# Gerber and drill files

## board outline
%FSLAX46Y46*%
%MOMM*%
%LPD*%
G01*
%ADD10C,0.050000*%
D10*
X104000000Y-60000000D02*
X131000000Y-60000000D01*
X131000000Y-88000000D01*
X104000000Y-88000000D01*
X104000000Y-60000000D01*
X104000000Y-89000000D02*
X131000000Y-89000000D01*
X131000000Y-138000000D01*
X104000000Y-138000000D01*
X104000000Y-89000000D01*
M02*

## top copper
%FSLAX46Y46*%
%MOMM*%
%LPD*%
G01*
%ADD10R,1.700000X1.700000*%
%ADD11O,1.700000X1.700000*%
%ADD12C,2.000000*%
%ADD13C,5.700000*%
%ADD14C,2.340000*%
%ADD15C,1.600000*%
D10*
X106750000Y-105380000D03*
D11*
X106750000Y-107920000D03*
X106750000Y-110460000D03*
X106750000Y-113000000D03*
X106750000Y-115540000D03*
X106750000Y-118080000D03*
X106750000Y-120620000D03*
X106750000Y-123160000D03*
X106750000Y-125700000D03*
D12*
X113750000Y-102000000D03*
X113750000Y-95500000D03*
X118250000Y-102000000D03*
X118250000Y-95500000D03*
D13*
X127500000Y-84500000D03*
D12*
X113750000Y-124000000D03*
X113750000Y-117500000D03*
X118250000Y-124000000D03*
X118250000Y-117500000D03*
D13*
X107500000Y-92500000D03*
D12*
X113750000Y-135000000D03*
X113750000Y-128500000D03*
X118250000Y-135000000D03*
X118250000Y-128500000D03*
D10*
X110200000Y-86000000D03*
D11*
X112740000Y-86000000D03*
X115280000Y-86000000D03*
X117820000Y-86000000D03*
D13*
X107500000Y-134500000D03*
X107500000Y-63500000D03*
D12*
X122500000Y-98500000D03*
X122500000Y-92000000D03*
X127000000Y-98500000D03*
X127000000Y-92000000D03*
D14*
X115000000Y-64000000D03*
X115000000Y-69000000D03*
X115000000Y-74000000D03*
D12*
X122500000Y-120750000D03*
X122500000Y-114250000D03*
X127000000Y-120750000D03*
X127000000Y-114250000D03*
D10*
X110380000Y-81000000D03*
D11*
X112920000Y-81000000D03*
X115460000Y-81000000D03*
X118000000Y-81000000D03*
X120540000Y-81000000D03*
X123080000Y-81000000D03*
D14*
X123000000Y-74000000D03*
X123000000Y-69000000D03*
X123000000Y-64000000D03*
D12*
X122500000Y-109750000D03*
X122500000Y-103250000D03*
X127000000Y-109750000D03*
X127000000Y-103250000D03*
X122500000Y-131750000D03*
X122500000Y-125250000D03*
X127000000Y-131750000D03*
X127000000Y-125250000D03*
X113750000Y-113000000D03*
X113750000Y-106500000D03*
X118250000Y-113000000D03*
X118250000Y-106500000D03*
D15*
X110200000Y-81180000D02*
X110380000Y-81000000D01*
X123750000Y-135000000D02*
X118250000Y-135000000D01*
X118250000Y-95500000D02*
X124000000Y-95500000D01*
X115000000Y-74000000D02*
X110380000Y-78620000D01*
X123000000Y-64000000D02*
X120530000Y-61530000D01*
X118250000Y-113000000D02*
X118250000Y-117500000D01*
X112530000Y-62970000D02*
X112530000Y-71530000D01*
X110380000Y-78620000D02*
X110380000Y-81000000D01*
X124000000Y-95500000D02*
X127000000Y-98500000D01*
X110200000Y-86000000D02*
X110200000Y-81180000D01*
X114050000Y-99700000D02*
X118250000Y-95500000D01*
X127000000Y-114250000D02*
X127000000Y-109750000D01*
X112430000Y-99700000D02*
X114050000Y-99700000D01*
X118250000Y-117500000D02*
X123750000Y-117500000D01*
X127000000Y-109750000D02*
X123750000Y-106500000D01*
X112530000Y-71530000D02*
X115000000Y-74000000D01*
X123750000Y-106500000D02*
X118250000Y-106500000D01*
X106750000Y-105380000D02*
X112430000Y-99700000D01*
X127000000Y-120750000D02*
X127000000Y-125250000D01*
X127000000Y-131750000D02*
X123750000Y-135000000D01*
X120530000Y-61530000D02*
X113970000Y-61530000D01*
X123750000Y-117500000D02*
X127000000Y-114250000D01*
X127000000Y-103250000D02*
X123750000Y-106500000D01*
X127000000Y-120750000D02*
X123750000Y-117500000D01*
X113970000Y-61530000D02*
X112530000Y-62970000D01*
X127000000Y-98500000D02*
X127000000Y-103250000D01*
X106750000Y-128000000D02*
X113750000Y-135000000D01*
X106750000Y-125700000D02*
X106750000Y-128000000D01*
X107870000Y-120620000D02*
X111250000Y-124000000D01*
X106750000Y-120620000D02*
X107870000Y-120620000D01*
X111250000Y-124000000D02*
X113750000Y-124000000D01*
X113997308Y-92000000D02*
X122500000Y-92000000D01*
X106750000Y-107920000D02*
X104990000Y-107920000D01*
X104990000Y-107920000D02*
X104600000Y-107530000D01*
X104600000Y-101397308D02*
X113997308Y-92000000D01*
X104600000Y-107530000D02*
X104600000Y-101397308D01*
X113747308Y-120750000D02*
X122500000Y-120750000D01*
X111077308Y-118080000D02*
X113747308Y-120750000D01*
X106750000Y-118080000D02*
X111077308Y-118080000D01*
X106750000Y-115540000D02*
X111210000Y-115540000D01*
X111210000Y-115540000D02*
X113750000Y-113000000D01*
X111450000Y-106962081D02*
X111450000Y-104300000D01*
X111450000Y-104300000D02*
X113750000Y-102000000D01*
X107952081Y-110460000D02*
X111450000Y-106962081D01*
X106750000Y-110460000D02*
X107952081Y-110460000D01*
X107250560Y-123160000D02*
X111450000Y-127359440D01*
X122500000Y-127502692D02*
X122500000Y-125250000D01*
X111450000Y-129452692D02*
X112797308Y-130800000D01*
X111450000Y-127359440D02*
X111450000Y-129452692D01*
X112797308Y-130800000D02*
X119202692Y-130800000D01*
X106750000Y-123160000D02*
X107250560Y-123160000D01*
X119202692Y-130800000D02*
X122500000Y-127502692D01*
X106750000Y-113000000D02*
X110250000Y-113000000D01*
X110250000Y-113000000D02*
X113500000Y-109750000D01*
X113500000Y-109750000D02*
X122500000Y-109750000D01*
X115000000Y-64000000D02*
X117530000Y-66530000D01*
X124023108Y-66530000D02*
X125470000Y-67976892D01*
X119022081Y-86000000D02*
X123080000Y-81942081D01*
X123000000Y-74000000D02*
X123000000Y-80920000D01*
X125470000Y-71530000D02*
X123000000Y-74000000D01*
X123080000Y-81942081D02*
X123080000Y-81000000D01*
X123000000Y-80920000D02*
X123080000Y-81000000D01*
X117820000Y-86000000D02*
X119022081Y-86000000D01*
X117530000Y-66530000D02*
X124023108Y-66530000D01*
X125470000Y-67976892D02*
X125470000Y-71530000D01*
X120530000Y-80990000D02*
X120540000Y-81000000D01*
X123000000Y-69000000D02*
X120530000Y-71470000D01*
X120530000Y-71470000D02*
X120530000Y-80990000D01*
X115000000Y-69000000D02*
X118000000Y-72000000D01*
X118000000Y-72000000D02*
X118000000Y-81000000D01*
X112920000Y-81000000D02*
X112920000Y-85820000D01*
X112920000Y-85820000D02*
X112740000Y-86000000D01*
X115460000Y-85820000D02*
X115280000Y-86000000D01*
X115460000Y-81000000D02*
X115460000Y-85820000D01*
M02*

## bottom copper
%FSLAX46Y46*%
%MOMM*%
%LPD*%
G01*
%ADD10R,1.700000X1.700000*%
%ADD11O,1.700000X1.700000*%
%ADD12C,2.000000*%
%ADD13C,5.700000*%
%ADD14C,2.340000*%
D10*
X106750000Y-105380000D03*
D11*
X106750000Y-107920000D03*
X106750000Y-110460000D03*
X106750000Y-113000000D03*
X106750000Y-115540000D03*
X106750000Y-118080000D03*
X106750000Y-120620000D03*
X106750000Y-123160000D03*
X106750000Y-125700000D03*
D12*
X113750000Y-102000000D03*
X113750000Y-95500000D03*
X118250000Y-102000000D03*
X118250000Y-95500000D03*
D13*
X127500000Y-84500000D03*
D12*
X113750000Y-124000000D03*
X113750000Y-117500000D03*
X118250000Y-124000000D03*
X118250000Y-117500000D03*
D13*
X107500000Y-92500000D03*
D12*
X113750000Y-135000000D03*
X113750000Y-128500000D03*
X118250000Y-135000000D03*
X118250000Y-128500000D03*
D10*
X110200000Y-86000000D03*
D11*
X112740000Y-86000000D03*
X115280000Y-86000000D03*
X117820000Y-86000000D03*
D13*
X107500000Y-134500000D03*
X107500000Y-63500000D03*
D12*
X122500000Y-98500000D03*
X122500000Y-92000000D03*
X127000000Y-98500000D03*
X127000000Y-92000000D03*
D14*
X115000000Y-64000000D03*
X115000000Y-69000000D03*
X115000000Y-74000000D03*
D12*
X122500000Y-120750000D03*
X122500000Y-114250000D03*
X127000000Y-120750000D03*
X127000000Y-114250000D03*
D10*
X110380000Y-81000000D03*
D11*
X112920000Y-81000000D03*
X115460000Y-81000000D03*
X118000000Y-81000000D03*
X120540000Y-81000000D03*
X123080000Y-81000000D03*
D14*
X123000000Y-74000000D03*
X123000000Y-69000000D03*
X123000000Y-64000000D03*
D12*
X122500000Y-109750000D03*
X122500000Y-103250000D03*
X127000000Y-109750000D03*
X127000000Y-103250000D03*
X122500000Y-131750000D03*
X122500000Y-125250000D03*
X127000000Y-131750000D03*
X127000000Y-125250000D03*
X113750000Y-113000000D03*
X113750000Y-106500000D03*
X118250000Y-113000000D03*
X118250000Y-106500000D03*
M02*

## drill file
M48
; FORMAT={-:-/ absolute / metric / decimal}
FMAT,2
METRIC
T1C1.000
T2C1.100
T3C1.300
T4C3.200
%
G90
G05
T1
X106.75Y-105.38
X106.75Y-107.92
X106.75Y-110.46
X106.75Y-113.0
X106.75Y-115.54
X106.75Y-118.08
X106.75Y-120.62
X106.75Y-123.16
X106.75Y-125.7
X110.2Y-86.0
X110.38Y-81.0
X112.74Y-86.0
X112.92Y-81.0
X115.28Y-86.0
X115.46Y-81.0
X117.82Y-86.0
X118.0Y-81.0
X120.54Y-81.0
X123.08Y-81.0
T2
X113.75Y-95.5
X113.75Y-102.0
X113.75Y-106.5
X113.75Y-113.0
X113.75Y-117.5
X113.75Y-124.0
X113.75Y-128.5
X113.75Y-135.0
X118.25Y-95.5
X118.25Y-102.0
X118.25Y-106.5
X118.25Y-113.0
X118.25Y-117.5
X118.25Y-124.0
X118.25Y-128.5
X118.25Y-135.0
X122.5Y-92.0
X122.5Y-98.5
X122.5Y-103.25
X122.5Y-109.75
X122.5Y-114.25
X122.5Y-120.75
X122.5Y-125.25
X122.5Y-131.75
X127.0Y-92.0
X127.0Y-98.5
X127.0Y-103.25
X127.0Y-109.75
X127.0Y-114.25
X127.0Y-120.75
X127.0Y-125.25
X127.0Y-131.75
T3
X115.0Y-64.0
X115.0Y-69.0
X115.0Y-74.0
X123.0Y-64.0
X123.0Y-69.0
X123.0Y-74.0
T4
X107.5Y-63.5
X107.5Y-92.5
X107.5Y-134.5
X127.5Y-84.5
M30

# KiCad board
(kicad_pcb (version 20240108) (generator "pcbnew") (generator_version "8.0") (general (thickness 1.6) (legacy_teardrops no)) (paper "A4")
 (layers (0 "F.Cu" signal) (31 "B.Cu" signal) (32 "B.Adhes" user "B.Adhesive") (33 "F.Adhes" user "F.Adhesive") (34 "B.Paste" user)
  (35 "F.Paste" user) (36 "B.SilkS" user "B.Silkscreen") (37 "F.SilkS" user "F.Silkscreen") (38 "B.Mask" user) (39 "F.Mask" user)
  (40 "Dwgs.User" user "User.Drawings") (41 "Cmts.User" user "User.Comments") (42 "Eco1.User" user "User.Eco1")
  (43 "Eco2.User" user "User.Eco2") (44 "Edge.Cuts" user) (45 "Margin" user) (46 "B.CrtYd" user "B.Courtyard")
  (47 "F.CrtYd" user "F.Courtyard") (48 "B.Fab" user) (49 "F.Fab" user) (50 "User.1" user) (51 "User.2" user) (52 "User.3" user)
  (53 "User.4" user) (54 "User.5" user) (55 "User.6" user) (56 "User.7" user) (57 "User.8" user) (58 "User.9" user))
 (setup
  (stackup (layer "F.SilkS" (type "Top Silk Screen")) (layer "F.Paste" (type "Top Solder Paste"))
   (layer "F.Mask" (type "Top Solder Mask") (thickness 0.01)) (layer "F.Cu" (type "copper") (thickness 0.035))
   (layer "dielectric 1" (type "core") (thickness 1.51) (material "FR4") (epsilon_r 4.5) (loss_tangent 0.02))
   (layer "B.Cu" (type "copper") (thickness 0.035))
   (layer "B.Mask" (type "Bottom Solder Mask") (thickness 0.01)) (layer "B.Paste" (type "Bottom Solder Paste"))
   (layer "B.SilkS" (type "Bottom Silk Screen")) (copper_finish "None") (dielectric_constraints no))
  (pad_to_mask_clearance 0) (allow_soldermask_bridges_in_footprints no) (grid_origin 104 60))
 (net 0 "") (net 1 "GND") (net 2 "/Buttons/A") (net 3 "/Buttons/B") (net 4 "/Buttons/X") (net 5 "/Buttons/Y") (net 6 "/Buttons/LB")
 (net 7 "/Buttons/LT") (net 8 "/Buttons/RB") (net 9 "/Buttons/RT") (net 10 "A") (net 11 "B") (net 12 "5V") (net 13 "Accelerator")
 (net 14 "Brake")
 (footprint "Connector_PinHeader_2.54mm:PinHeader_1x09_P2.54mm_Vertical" (layer "F.Cu") (at 106.75 105.38)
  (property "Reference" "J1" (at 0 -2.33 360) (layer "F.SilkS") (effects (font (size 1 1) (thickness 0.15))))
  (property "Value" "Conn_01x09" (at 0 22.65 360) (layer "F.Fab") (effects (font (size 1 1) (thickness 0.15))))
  (pad "1" thru_hole rect (at 0 0) (size 1.7 1.7) (drill 1) (layers "*.Cu" "*.Mask") (remove_unused_layers no) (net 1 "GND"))
  (pad "2" thru_hole oval (at 0 2.54) (size 1.7 1.7) (drill 1) (layers "*.Cu" "*.Mask") (remove_unused_layers no) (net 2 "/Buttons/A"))
  (pad "3" thru_hole oval (at 0 5.08) (size 1.7 1.7) (drill 1) (layers "*.Cu" "*.Mask") (remove_unused_layers no) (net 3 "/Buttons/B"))
  (pad "4" thru_hole oval (at 0 7.62) (size 1.7 1.7) (drill 1) (layers "*.Cu" "*.Mask") (remove_unused_layers no) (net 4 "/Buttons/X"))
  (pad "5" thru_hole oval (at 0 10.16) (size 1.7 1.7) (drill 1) (layers "*.Cu" "*.Mask") (remove_unused_layers no) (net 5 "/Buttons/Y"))
  (pad "6" thru_hole oval (at 0 12.7) (size 1.7 1.7) (drill 1) (layers "*.Cu" "*.Mask") (remove_unused_layers no) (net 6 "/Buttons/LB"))
  (pad "7" thru_hole oval (at 0 15.24) (size 1.7 1.7) (drill 1) (layers "*.Cu" "*.Mask") (remove_unused_layers no) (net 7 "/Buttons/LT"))
  (pad "8" thru_hole oval (at 0 17.78) (size 1.7 1.7) (drill 1) (layers "*.Cu" "*.Mask") (remove_unused_layers no) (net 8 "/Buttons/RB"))
  (pad "9" thru_hole oval (at 0 20.32) (size 1.7 1.7) (drill 1) (layers "*.Cu" "*.Mask") (remove_unused_layers no) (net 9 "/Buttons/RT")))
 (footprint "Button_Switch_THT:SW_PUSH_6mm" (layer "F.Cu") (at 113.75 102 90)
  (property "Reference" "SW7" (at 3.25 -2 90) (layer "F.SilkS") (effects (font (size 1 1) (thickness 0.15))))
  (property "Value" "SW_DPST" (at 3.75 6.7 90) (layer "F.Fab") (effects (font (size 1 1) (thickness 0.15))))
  (pad "1" thru_hole circle (at 0 0 180) (size 2 2) (drill 1.1) (layers "*.Cu" "*.Mask") (remove_unused_layers no) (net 3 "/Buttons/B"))
  (pad "1" thru_hole circle (at 6.5 0 180) (size 2 2) (drill 1.1) (layers "*.Cu" "*.Mask") (remove_unused_layers no) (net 3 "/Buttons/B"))
  (pad "2" thru_hole circle (at 0 4.5 180) (size 2 2) (drill 1.1) (layers "*.Cu" "*.Mask") (remove_unused_layers no) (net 1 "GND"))
  (pad "2" thru_hole circle (at 6.5 4.5 180) (size 2 2) (drill 1.1) (layers "*.Cu" "*.Mask") (remove_unused_layers no) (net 1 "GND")))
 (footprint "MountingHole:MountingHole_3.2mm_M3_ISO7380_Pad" (layer "F.Cu") (at 127.5 84.5)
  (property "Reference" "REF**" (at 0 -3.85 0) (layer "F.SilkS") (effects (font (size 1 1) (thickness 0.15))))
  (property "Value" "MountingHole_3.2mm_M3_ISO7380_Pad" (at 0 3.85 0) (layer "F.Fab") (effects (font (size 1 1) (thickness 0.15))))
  (pad "1" thru_hole circle (at 0 0) (size 5.7 5.7) (drill 3.2) (layers "*.Cu" "*.Mask") (remove_unused_layers no)))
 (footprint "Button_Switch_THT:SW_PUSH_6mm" (layer "F.Cu") (at 113.75 124 90)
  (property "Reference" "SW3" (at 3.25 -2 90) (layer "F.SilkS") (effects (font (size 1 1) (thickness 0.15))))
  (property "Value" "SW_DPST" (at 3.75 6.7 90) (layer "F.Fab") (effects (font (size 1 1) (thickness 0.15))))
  (pad "1" thru_hole circle (at 0 0 180) (size 2 2) (drill 1.1) (layers "*.Cu" "*.Mask") (remove_unused_layers no) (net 7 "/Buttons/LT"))
  (pad "1" thru_hole circle (at 6.5 0 180) (size 2 2) (drill 1.1) (layers "*.Cu" "*.Mask") (remove_unused_layers no) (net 7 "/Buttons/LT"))
  (pad "2" thru_hole circle (at 0 4.5 180) (size 2 2) (drill 1.1) (layers "*.Cu" "*.Mask") (remove_unused_layers no) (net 1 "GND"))
  (pad "2" thru_hole circle (at 6.5 4.5 180) (size 2 2) (drill 1.1) (layers "*.Cu" "*.Mask") (remove_unused_layers no) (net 1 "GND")))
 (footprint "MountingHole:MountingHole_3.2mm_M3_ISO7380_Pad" (layer "F.Cu") (at 107.5 92.5)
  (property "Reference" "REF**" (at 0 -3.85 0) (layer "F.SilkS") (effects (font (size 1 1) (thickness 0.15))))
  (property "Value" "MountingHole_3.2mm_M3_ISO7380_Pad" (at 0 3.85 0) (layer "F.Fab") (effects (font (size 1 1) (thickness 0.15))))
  (pad "1" thru_hole circle (at 0 0) (size 5.7 5.7) (drill 3.2) (layers "*.Cu" "*.Mask") (remove_unused_layers no)))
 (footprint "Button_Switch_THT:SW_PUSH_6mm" (layer "F.Cu") (at 113.75 135 90)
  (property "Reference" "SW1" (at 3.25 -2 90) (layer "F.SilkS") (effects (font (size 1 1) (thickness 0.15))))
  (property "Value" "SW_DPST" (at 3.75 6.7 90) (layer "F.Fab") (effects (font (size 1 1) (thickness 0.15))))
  (pad "1" thru_hole circle (at 0 0 180) (size 2 2) (drill 1.1) (layers "*.Cu" "*.Mask") (remove_unused_layers no) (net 9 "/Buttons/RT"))
  (pad "1" thru_hole circle (at 6.5 0 180) (size 2 2) (drill 1.1) (layers "*.Cu" "*.Mask") (remove_unused_layers no) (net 9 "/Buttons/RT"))
  (pad "2" thru_hole circle (at 0 4.5 180) (size 2 2) (drill 1.1) (layers "*.Cu" "*.Mask") (remove_unused_layers no) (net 1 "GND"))
  (pad "2" thru_hole circle (at 6.5 4.5 180) (size 2 2) (drill 1.1) (layers "*.Cu" "*.Mask") (remove_unused_layers no) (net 1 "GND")))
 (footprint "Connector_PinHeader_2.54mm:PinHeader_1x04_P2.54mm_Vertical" (layer "F.Cu") (at 110.2 86 90)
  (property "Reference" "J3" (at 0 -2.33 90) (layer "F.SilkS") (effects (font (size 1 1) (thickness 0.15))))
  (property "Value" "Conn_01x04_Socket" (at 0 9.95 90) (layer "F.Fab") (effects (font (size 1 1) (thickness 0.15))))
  (pad "1" thru_hole rect (at 0 0 90) (size 1.7 1.7) (drill 1) (layers "*.Cu" "*.Mask") (remove_unused_layers no) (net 1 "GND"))
  (pad "2" thru_hole oval (at 0 2.54 90) (size 1.7 1.7) (drill 1) (layers "*.Cu" "*.Mask") (remove_unused_layers no) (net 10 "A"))
  (pad "3" thru_hole oval (at 0 5.08 90) (size 1.7 1.7) (drill 1) (layers "*.Cu" "*.Mask") (remove_unused_layers no) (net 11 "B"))
  (pad "4" thru_hole oval (at 0 7.62 90) (size 1.7 1.7) (drill 1) (layers "*.Cu" "*.Mask") (remove_unused_layers no) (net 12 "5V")))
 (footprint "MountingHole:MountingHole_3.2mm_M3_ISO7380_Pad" (layer "F.Cu") (at 107.5 134.5)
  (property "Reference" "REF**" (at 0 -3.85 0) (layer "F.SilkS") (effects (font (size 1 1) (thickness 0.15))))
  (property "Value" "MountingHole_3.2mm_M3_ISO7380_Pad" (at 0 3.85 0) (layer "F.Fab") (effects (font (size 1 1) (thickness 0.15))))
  (pad "1" thru_hole circle (at 0 0) (size 5.7 5.7) (drill 3.2) (layers "*.Cu" "*.Mask") (remove_unused_layers no)))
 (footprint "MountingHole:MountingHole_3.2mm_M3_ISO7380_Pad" (layer "F.Cu") (at 107.5 63.5)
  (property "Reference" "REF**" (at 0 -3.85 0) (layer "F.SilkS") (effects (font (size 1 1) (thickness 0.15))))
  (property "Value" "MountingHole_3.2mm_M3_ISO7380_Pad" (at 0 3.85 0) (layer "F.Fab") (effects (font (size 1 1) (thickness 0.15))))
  (pad "1" thru_hole circle (at 0 0) (size 5.7 5.7) (drill 3.2) (layers "*.Cu" "*.Mask") (remove_unused_layers no)))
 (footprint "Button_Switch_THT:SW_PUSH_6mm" (layer "F.Cu") (at 122.5 98.5 90)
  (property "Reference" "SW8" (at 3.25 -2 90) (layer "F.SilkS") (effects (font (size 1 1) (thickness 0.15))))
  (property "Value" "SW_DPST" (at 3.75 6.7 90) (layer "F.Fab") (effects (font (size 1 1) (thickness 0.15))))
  (pad "1" thru_hole circle (at 0 0 180) (size 2 2) (drill 1.1) (layers "*.Cu" "*.Mask") (remove_unused_layers no) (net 2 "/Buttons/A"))
  (pad "1" thru_hole circle (at 6.5 0 180) (size 2 2) (drill 1.1) (layers "*.Cu" "*.Mask") (remove_unused_layers no) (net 2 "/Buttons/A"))
  (pad "2" thru_hole circle (at 0 4.5 180) (size 2 2) (drill 1.1) (layers "*.Cu" "*.Mask") (remove_unused_layers no) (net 1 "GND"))
  (pad "2" thru_hole circle (at 6.5 4.5 180) (size 2 2) (drill 1.1) (layers "*.Cu" "*.Mask") (remove_unused_layers no) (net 1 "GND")))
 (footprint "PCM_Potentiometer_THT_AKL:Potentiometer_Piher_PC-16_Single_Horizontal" (layer "F.Cu") (at 115 64 180)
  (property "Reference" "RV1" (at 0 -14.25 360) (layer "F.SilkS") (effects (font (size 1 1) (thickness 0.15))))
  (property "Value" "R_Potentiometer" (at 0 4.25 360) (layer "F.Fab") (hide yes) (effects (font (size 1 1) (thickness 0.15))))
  (pad "1" thru_hole circle (at 0 0 180) (size 2.34 2.34) (drill 1.3) (layers "*.Cu" "*.Mask") (remove_unused_layers no) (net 12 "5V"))
  (pad "2" thru_hole circle (at 0 -5 180) (size 2.34 2.34) (drill 1.3) (layers "*.Cu" "*.Mask") (remove_unused_layers no)
   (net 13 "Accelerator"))
  (pad "3" thru_hole circle (at 0 -10 180) (size 2.34 2.34) (drill 1.3) (layers "*.Cu" "*.Mask") (remove_unused_layers no) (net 1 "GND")))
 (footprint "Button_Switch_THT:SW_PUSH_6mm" (layer "F.Cu") (at 122.5 120.75 90)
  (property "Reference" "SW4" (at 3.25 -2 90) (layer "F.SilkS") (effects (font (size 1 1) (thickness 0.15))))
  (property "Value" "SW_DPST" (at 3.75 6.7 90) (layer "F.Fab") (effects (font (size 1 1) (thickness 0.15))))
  (pad "1" thru_hole circle (at 0 0 180) (size 2 2) (drill 1.1) (layers "*.Cu" "*.Mask") (remove_unused_layers no) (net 6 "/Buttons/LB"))
  (pad "1" thru_hole circle (at 6.5 0 180) (size 2 2) (drill 1.1) (layers "*.Cu" "*.Mask") (remove_unused_layers no) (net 6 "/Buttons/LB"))
  (pad "2" thru_hole circle (at 0 4.5 180) (size 2 2) (drill 1.1) (layers "*.Cu" "*.Mask") (remove_unused_layers no) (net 1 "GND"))
  (pad "2" thru_hole circle (at 6.5 4.5 180) (size 2 2) (drill 1.1) (layers "*.Cu" "*.Mask") (remove_unused_layers no) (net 1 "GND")))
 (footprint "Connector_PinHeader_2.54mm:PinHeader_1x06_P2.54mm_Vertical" (layer "F.Cu") (at 110.38 81 90)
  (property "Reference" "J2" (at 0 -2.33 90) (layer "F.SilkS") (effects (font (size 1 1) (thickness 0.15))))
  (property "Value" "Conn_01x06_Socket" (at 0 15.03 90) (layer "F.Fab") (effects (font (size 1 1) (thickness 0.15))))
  (pad "1" thru_hole rect (at 0 0 90) (size 1.7 1.7) (drill 1) (layers "*.Cu" "*.Mask") (remove_unused_layers no) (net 1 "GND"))
  (pad "2" thru_hole oval (at 0 2.54 90) (size 1.7 1.7) (drill 1) (layers "*.Cu" "*.Mask") (remove_unused_layers no) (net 10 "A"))
  (pad "3" thru_hole oval (at 0 5.08 90) (size 1.7 1.7) (drill 1) (layers "*.Cu" "*.Mask") (remove_unused_layers no) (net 11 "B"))
  (pad "4" thru_hole oval (at 0 7.62 90) (size 1.7 1.7) (drill 1) (layers "*.Cu" "*.Mask") (remove_unused_layers no) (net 13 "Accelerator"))
  (pad "5" thru_hole oval (at 0 10.16 90) (size 1.7 1.7) (drill 1) (layers "*.Cu" "*.Mask") (remove_unused_layers no) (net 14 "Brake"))
  (pad "6" thru_hole oval (at 0 12.7 90) (size 1.7 1.7) (drill 1) (layers "*.Cu" "*.Mask") (remove_unused_layers no) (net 12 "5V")))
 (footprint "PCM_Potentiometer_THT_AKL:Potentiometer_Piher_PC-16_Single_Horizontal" (layer "F.Cu") (at 123 74)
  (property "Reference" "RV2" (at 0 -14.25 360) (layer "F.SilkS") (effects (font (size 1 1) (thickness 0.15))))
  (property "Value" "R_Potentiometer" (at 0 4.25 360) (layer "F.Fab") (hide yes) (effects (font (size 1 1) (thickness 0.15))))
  (pad "1" thru_hole circle (at 0 0) (size 2.34 2.34) (drill 1.3) (layers "*.Cu" "*.Mask") (remove_unused_layers no) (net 12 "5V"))
  (pad "2" thru_hole circle (at 0 -5) (size 2.34 2.34) (drill 1.3) (layers "*.Cu" "*.Mask") (remove_unused_layers no) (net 14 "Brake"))
  (pad "3" thru_hole circle (at 0 -10) (size 2.34 2.34) (drill 1.3) (layers "*.Cu" "*.Mask") (remove_unused_layers no) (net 1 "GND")))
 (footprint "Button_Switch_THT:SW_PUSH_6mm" (layer "F.Cu") (at 122.5 109.75 90)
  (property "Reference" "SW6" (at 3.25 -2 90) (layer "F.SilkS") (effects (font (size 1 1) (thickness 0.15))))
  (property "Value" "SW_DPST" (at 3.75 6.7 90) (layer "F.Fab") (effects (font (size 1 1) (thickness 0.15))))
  (pad "1" thru_hole circle (at 0 0 180) (size 2 2) (drill 1.1) (layers "*.Cu" "*.Mask") (remove_unused_layers no) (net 4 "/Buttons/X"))
  (pad "1" thru_hole circle (at 6.5 0 180) (size 2 2) (drill 1.1) (layers "*.Cu" "*.Mask") (remove_unused_layers no) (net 4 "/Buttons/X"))
  (pad "2" thru_hole circle (at 0 4.5 180) (size 2 2) (drill 1.1) (layers "*.Cu" "*.Mask") (remove_unused_layers no) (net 1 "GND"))
  (pad "2" thru_hole circle (at 6.5 4.5 180) (size 2 2) (drill 1.1) (layers "*.Cu" "*.Mask") (remove_unused_layers no) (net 1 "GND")))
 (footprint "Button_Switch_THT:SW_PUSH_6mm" (layer "F.Cu") (at 122.5 131.75 90)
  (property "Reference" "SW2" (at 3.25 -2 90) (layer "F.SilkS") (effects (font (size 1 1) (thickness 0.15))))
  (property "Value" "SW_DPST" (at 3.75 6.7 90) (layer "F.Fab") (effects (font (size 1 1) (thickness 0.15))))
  (pad "1" thru_hole circle (at 0 0 180) (size 2 2) (drill 1.1) (layers "*.Cu" "*.Mask") (remove_unused_layers no) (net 8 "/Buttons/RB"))
  (pad "1" thru_hole circle (at 6.5 0 180) (size 2 2) (drill 1.1) (layers "*.Cu" "*.Mask") (remove_unused_layers no) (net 8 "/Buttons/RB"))
  (pad "2" thru_hole circle (at 0 4.5 180) (size 2 2) (drill 1.1) (layers "*.Cu" "*.Mask") (remove_unused_layers no) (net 1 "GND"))
  (pad "2" thru_hole circle (at 6.5 4.5 180) (size 2 2) (drill 1.1) (layers "*.Cu" "*.Mask") (remove_unused_layers no) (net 1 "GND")))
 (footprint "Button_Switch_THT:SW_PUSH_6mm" (layer "F.Cu") (at 113.75 113 90)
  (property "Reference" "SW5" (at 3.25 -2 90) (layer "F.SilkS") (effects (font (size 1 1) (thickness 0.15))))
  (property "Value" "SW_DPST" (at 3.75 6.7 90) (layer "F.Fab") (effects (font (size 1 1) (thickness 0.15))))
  (pad "1" thru_hole circle (at 0 0 180) (size 2 2) (drill 1.1) (layers "*.Cu" "*.Mask") (remove_unused_layers no) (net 5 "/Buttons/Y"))
  (pad "1" thru_hole circle (at 6.5 0 180) (size 2 2) (drill 1.1) (layers "*.Cu" "*.Mask") (remove_unused_layers no) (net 5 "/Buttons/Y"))
  (pad "2" thru_hole circle (at 0 4.5 180) (size 2 2) (drill 1.1) (layers "*.Cu" "*.Mask") (remove_unused_layers no) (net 1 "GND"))
  (pad "2" thru_hole circle (at 6.5 4.5 180) (size 2 2) (drill 1.1) (layers "*.Cu" "*.Mask") (remove_unused_layers no) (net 1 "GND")))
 (gr_rect (start 104 60) (end 131 88) (stroke (width 0.05) (type default)) (fill none) (layer "Edge.Cuts"))
 (gr_rect (start 104 89) (end 131 138) (stroke (width 0.05) (type default)) (fill none) (layer "Edge.Cuts"))
 (segment (start 110.2 81.18) (end 110.38 81) (width 1.6) (layer "F.Cu") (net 1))
 (segment (start 123.75 135) (end 118.25 135) (width 1.6) (layer "F.Cu") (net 1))
 (segment (start 118.25 95.5) (end 124 95.5) (width 1.6) (layer "F.Cu") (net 1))
 (segment (start 115 74) (end 110.38 78.62) (width 1.6) (layer "F.Cu") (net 1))
 (segment (start 123 64) (end 120.53 61.53) (width 1.6) (layer "F.Cu") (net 1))
 (segment (start 118.25 113) (end 118.25 117.5) (width 1.6) (layer "F.Cu") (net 1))
 (segment (start 112.53 62.97) (end 112.53 71.53) (width 1.6) (layer "F.Cu") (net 1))
 (segment (start 110.38 78.62) (end 110.38 81) (width 1.6) (layer "F.Cu") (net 1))
 (segment (start 124 95.5) (end 127 98.5) (width 1.6) (layer "F.Cu") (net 1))
 (segment (start 110.2 86) (end 110.2 81.18) (width 1.6) (layer "F.Cu") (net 1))
 (segment (start 114.05 99.7) (end 118.25 95.5) (width 1.6) (layer "F.Cu") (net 1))
 (segment (start 127 114.25) (end 127 109.75) (width 1.6) (layer "F.Cu") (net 1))
 (segment (start 112.43 99.7) (end 114.05 99.7) (width 1.6) (layer "F.Cu") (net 1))
 (segment (start 118.25 117.5) (end 123.75 117.5) (width 1.6) (layer "F.Cu") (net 1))
 (segment (start 127 109.75) (end 123.75 106.5) (width 1.6) (layer "F.Cu") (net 1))
 (segment (start 112.53 71.53) (end 115 74) (width 1.6) (layer "F.Cu") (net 1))
 (segment (start 123.75 106.5) (end 118.25 106.5) (width 1.6) (layer "F.Cu") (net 1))
 (segment (start 106.75 105.38) (end 112.43 99.7) (width 1.6) (layer "F.Cu") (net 1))
 (segment (start 127 120.75) (end 127 125.25) (width 1.6) (layer "F.Cu") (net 1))
 (segment (start 127 131.75) (end 123.75 135) (width 1.6) (layer "F.Cu") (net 1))
 (segment (start 120.53 61.53) (end 113.97 61.53) (width 1.6) (layer "F.Cu") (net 1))
 (segment (start 123.75 117.5) (end 127 114.25) (width 1.6) (layer "F.Cu") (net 1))
 (segment (start 127 103.25) (end 123.75 106.5) (width 1.6) (layer "F.Cu") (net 1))
 (segment (start 127 120.75) (end 123.75 117.5) (width 1.6) (layer "F.Cu") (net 1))
 (segment (start 113.97 61.53) (end 112.53 62.97) (width 1.6) (layer "F.Cu") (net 1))
 (segment (start 127 98.5) (end 127 103.25) (width 1.6) (layer "F.Cu") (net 1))
 (segment (start 106.75 128) (end 113.75 135) (width 1.6) (layer "F.Cu") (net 9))
 (segment (start 106.75 125.7) (end 106.75 128) (width 1.6) (layer "F.Cu") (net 9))
 (segment (start 107.87 120.62) (end 111.25 124) (width 1.6) (layer "F.Cu") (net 7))
 (segment (start 106.75 120.62) (end 107.87 120.62) (width 1.6) (layer "F.Cu") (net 7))
 (segment (start 111.25 124) (end 113.75 124) (width 1.6) (layer "F.Cu") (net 7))
 (segment (start 113.997308 92) (end 122.5 92) (width 1.6) (layer "F.Cu") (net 2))
 (segment (start 106.75 107.92) (end 104.99 107.92) (width 1.6) (layer "F.Cu") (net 2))
 (segment (start 104.99 107.92) (end 104.6 107.53) (width 1.6) (layer "F.Cu") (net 2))
 (segment (start 104.6 101.397308) (end 113.997308 92) (width 1.6) (layer "F.Cu") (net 2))
 (segment (start 104.6 107.53) (end 104.6 101.397308) (width 1.6) (layer "F.Cu") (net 2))
 (segment (start 113.747308 120.75) (end 122.5 120.75) (width 1.6) (layer "F.Cu") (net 6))
 (segment (start 111.077308 118.08) (end 113.747308 120.75) (width 1.6) (layer "F.Cu") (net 6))
 (segment (start 106.75 118.08) (end 111.077308 118.08) (width 1.6) (layer "F.Cu") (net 6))
 (segment (start 106.75 115.54) (end 111.21 115.54) (width 1.6) (layer "F.Cu") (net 5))
 (segment (start 111.21 115.54) (end 113.75 113) (width 1.6) (layer "F.Cu") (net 5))
 (segment (start 111.45 106.962081) (end 111.45 104.3) (width 1.6) (layer "F.Cu") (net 3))
 (segment (start 111.45 104.3) (end 113.75 102) (width 1.6) (layer "F.Cu") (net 3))
 (segment (start 107.952081 110.46) (end 111.45 106.962081) (width 1.6) (layer "F.Cu") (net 3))
 (segment (start 106.75 110.46) (end 107.952081 110.46) (width 1.6) (layer "F.Cu") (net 3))
 (segment (start 107.25056 123.16) (end 111.45 127.35944) (width 1.6) (layer "F.Cu") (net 8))
 (segment (start 122.5 127.502692) (end 122.5 125.25) (width 1.6) (layer "F.Cu") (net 8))
 (segment (start 111.45 129.452692) (end 112.797308 130.8) (width 1.6) (layer "F.Cu") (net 8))
 (segment (start 111.45 127.35944) (end 111.45 129.452692) (width 1.6) (layer "F.Cu") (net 8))
 (segment (start 112.797308 130.8) (end 119.202692 130.8) (width 1.6) (layer "F.Cu") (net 8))
 (segment (start 106.75 123.16) (end 107.25056 123.16) (width 1.6) (layer "F.Cu") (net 8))
 (segment (start 119.202692 130.8) (end 122.5 127.502692) (width 1.6) (layer "F.Cu") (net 8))
 (segment (start 106.75 113) (end 110.25 113) (width 1.6) (layer "F.Cu") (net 4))
 (segment (start 110.25 113) (end 113.5 109.75) (width 1.6) (layer "F.Cu") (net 4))
 (segment (start 113.5 109.75) (end 122.5 109.75) (width 1.6) (layer "F.Cu") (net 4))
 (segment (start 115 64) (end 117.53 66.53) (width 1.6) (layer "F.Cu") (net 12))
 (segment (start 124.023108 66.53) (end 125.47 67.976892) (width 1.6) (layer "F.Cu") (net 12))
 (segment (start 119.022081 86) (end 123.08 81.942081) (width 1.6) (layer "F.Cu") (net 12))
 (segment (start 123 74) (end 123 80.92) (width 1.6) (layer "F.Cu") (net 12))
 (segment (start 125.47 71.53) (end 123 74) (width 1.6) (layer "F.Cu") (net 12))
 (segment (start 123.08 81.942081) (end 123.08 81) (width 1.6) (layer "F.Cu") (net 12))
 (segment (start 123 80.92) (end 123.08 81) (width 1.6) (layer "F.Cu") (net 12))
 (segment (start 117.82 86) (end 119.022081 86) (width 1.6) (layer "F.Cu") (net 12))
 (segment (start 117.53 66.53) (end 124.023108 66.53) (width 1.6) (layer "F.Cu") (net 12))
 (segment (start 125.47 67.976892) (end 125.47 71.53) (width 1.6) (layer "F.Cu") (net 12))
 (segment (start 120.53 80.99) (end 120.54 81) (width 1.6) (layer "F.Cu") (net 14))
 (segment (start 123 69) (end 120.53 71.47) (width 1.6) (layer "F.Cu") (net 14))
 (segment (start 120.53 71.47) (end 120.53 80.99) (width 1.6) (layer "F.Cu") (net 14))
 (segment (start 115 69) (end 118 72) (width 1.6) (layer "F.Cu") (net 13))
 (segment (start 118 72) (end 118 81) (width 1.6) (layer "F.Cu") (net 13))
 (segment (start 112.92 81) (end 112.92 85.82) (width 1.6) (layer "F.Cu") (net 10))
 (segment (start 112.92 85.82) (end 112.74 86) (width 1.6) (layer "F.Cu") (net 10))
 (segment (start 115.46 85.82) (end 115.28 86) (width 1.6) (layer "F.Cu") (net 11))
 (segment (start 115.46 81) (end 115.46 85.82) (width 1.6) (layer "F.Cu") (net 11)))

